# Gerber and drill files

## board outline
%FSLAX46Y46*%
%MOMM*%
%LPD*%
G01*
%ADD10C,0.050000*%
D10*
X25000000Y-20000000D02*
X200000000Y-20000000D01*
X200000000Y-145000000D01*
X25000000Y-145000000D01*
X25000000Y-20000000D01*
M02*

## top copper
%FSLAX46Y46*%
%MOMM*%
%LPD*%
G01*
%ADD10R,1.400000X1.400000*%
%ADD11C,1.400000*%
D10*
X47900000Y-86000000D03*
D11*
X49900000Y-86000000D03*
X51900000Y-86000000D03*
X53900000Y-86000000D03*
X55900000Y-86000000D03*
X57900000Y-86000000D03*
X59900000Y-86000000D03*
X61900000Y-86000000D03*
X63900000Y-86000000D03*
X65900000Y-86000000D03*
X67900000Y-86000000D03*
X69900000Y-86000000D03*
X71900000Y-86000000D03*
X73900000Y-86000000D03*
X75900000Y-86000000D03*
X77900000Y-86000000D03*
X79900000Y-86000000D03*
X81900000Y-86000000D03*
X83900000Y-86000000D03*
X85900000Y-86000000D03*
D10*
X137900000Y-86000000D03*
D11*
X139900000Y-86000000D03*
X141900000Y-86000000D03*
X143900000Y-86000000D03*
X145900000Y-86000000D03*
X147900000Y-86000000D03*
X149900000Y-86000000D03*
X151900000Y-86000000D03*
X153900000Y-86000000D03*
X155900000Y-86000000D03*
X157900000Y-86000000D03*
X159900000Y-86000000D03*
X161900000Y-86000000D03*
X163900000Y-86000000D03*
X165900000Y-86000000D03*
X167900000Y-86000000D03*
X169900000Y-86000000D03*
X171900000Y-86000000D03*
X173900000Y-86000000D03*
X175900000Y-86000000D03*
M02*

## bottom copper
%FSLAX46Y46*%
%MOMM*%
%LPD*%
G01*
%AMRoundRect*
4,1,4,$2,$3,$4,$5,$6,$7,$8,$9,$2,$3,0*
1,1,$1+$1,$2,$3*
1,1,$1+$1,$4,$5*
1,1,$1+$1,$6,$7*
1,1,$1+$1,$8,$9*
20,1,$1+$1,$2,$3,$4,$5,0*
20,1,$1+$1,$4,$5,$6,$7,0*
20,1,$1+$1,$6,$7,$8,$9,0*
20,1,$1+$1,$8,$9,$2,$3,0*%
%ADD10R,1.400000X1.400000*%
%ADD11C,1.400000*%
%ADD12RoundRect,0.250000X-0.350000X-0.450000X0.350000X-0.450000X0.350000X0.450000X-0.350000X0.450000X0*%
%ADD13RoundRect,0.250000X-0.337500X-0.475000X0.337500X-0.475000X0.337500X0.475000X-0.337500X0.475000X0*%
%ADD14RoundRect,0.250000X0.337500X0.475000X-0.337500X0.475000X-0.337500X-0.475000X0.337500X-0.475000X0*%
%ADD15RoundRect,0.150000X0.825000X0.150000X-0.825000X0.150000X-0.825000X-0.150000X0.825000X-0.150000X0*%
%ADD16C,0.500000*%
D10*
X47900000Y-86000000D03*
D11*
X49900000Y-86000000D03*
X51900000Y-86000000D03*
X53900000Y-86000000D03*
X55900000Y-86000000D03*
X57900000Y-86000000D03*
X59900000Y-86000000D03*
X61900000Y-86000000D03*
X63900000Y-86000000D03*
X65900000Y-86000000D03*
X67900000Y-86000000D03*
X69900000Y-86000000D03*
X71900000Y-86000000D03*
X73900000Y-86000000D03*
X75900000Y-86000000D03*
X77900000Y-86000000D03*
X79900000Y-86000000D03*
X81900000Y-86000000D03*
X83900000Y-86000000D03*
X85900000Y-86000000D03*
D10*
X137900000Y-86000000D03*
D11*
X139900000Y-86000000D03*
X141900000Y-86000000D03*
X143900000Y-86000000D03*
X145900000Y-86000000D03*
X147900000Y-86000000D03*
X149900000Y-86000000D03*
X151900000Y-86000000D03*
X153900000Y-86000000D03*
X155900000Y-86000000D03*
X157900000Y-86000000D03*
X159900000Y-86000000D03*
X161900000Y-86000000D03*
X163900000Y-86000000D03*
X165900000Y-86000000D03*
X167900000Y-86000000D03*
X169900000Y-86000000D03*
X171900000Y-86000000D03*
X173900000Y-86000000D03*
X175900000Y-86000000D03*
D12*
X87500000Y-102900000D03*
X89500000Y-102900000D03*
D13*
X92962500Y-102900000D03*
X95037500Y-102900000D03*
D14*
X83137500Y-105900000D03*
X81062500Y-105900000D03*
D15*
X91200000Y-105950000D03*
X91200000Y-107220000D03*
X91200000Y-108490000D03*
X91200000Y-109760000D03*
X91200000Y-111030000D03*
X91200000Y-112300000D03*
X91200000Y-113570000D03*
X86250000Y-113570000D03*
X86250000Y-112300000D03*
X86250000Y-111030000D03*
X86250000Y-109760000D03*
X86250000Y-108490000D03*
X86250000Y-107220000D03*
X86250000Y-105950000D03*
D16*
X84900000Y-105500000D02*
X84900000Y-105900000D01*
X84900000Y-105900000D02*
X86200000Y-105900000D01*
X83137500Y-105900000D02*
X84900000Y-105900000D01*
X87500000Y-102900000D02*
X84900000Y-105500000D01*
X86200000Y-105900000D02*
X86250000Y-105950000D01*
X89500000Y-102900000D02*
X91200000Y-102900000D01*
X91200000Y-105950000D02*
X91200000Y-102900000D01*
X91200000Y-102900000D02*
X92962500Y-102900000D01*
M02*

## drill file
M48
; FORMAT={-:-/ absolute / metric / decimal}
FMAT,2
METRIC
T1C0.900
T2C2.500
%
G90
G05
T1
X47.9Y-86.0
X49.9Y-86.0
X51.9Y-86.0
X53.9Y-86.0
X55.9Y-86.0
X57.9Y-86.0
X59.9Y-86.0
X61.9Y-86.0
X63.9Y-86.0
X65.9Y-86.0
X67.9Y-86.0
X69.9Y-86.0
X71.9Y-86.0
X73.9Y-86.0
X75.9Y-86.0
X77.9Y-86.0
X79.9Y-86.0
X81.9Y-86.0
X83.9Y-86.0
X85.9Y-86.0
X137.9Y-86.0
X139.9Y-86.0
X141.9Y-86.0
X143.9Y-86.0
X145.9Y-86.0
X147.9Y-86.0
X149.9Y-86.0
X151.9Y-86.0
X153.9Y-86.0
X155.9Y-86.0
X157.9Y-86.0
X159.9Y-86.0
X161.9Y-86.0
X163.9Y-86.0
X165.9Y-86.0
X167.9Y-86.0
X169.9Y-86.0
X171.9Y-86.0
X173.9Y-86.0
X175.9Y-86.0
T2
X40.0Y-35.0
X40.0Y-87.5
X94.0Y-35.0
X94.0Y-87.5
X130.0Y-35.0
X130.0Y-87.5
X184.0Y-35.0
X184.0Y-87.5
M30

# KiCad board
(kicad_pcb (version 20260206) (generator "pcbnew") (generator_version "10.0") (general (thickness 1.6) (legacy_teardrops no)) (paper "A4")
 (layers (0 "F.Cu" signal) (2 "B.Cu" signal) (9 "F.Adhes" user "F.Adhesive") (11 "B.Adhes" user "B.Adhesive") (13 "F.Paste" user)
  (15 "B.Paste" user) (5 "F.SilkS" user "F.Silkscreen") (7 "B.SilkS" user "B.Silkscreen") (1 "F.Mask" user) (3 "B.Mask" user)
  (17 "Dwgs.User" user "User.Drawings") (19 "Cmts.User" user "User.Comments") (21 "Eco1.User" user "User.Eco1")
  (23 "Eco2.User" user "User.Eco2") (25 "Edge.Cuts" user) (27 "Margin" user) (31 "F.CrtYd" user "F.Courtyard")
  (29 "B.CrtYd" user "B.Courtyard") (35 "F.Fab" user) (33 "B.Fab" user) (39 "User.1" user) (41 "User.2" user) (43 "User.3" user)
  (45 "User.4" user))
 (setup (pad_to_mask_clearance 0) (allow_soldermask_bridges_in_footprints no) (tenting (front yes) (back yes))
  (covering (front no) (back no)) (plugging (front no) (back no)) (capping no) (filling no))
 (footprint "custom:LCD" (layer "F.Cu") (at 66.9 86)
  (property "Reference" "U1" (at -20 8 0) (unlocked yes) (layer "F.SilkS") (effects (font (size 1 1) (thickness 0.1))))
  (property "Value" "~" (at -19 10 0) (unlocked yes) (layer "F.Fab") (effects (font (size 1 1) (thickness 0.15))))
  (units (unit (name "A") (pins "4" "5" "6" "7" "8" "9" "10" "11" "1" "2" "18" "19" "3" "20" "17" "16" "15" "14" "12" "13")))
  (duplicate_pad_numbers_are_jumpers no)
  (pad "" np_thru_hole circle (at -26.9 -51) (size 2.5 2.5) (drill 2.5) (layers "*.Cu" "*.Mask") (thermal_bridge_angle 90))
  (pad "" np_thru_hole circle (at -26.9 1.5) (size 2.5 2.5) (drill 2.5) (layers "*.Cu" "*.Mask") (thermal_bridge_angle 90))
  (pad "" np_thru_hole circle (at 27.1 -51) (size 2.5 2.5) (drill 2.5) (layers "*.Cu" "*.Mask") (thermal_bridge_angle 90))
  (pad "" np_thru_hole circle (at 27.1 1.5) (size 2.5 2.5) (drill 2.5) (layers "*.Cu" "*.Mask") (thermal_bridge_angle 90))
  (pad "1" thru_hole rect (at -19 0) (size 1.4 1.4) (drill 0.9) (layers "*.Cu" "*.Mask") (remove_unused_layers no)
   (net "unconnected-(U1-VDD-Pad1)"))
  (pad "2" thru_hole circle (at -17 0) (size 1.4 1.4) (drill 0.9) (layers "*.Cu" "*.Mask") (remove_unused_layers no)
   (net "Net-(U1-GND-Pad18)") (thermal_bridge_angle 90))
  (pad "3" thru_hole circle (at -15 0) (size 1.4 1.4) (drill 0.9) (layers "*.Cu" "*.Mask") (remove_unused_layers no)
   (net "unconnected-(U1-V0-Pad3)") (thermal_bridge_angle 90))
  (pad "4" thru_hole circle (at -13 0) (size 1.4 1.4) (drill 0.9) (layers "*.Cu" "*.Mask") (remove_unused_layers no)
   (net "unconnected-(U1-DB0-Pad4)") (thermal_bridge_angle 90))
  (pad "5" thru_hole circle (at -11 0) (size 1.4 1.4) (drill 0.9) (layers "*.Cu" "*.Mask") (remove_unused_layers no)
   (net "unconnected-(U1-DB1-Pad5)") (thermal_bridge_angle 90))
  (pad "6" thru_hole circle (at -9 0) (size 1.4 1.4) (drill 0.9) (layers "*.Cu" "*.Mask") (remove_unused_layers no)
   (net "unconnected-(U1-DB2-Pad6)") (thermal_bridge_angle 90))
  (pad "7" thru_hole circle (at -7 0) (size 1.4 1.4) (drill 0.9) (layers "*.Cu" "*.Mask") (remove_unused_layers no)
   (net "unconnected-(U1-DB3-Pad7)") (thermal_bridge_angle 90))
  (pad "8" thru_hole circle (at -5 0) (size 1.4 1.4) (drill 0.9) (layers "*.Cu" "*.Mask") (remove_unused_layers no)
   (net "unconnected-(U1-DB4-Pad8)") (thermal_bridge_angle 90))
  (pad "9" thru_hole circle (at -3 0) (size 1.4 1.4) (drill 0.9) (layers "*.Cu" "*.Mask") (remove_unused_layers no)
   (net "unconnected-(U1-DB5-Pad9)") (thermal_bridge_angle 90))
  (pad "10" thru_hole circle (at -1 0) (size 1.4 1.4) (drill 0.9) (layers "*.Cu" "*.Mask") (remove_unused_layers no)
   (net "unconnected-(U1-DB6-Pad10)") (thermal_bridge_angle 90))
  (pad "11" thru_hole circle (at 1 0) (size 1.4 1.4) (drill 0.9) (layers "*.Cu" "*.Mask") (remove_unused_layers no)
   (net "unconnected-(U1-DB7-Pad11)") (thermal_bridge_angle 90))
  (pad "12" thru_hole circle (at 3 0) (size 1.4 1.4) (drill 0.9) (layers "*.Cu" "*.Mask") (remove_unused_layers no)
   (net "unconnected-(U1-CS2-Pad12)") (thermal_bridge_angle 90))
  (pad "13" thru_hole circle (at 5 0) (size 1.4 1.4) (drill 0.9) (layers "*.Cu" "*.Mask") (remove_unused_layers no)
   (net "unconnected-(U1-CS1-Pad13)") (thermal_bridge_angle 90))
  (pad "14" thru_hole circle (at 7 0) (size 1.4 1.4) (drill 0.9) (layers "*.Cu" "*.Mask") (remove_unused_layers no)
   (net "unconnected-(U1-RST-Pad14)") (thermal_bridge_angle 90))
  (pad "15" thru_hole circle (at 9 0) (size 1.4 1.4) (drill 0.9) (layers "*.Cu" "*.Mask") (remove_unused_layers no)
   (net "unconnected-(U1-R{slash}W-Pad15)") (thermal_bridge_angle 90))
  (pad "16" thru_hole circle (at 11 0) (size 1.4 1.4) (drill 0.9) (layers "*.Cu" "*.Mask") (remove_unused_layers no)
   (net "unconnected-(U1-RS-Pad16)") (thermal_bridge_angle 90))
  (pad "17" thru_hole circle (at 13 0) (size 1.4 1.4) (drill 0.9) (layers "*.Cu" "*.Mask") (remove_unused_layers no)
   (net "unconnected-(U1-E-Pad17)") (thermal_bridge_angle 90))
  (pad "18" thru_hole circle (at 15 0) (size 1.4 1.4) (drill 0.9) (layers "*.Cu" "*.Mask") (remove_unused_layers no)
   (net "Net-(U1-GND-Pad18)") (thermal_bridge_angle 90))
  (pad "19" thru_hole circle (at 17 0) (size 1.4 1.4) (drill 0.9) (layers "*.Cu" "*.Mask") (remove_unused_layers no)
   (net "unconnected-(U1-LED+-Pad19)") (thermal_bridge_angle 90))
  (pad "20" thru_hole circle (at 19 0) (size 1.4 1.4) (drill 0.9) (layers "*.Cu" "*.Mask") (remove_unused_layers no)
   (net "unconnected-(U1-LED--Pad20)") (thermal_bridge_angle 90)))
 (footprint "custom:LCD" (layer "F.Cu") (at 156.9 86)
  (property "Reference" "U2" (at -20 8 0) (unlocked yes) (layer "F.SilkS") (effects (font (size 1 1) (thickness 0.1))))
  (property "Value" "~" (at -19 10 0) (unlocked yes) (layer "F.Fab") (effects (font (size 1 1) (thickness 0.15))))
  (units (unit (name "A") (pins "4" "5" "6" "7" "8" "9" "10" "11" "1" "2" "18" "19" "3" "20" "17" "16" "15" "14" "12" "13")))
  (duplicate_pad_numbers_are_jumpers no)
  (pad "" np_thru_hole circle (at -26.9 -51) (size 2.5 2.5) (drill 2.5) (layers "*.Cu" "*.Mask") (thermal_bridge_angle 90))
  (pad "" np_thru_hole circle (at -26.9 1.5) (size 2.5 2.5) (drill 2.5) (layers "*.Cu" "*.Mask") (thermal_bridge_angle 90))
  (pad "" np_thru_hole circle (at 27.1 -51) (size 2.5 2.5) (drill 2.5) (layers "*.Cu" "*.Mask") (thermal_bridge_angle 90))
  (pad "" np_thru_hole circle (at 27.1 1.5) (size 2.5 2.5) (drill 2.5) (layers "*.Cu" "*.Mask") (thermal_bridge_angle 90))
  (pad "1" thru_hole rect (at -19 0) (size 1.4 1.4) (drill 0.9) (layers "*.Cu" "*.Mask") (remove_unused_layers no)
   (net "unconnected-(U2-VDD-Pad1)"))
  (pad "2" thru_hole circle (at -17 0) (size 1.4 1.4) (drill 0.9) (layers "*.Cu" "*.Mask") (remove_unused_layers no)
   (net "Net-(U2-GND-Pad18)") (thermal_bridge_angle 90))
  (pad "3" thru_hole circle (at -15 0) (size 1.4 1.4) (drill 0.9) (layers "*.Cu" "*.Mask") (remove_unused_layers no)
   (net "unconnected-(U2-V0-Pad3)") (thermal_bridge_angle 90))
  (pad "4" thru_hole circle (at -13 0) (size 1.4 1.4) (drill 0.9) (layers "*.Cu" "*.Mask") (remove_unused_layers no)
   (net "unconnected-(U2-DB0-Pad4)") (thermal_bridge_angle 90))
  (pad "5" thru_hole circle (at -11 0) (size 1.4 1.4) (drill 0.9) (layers "*.Cu" "*.Mask") (remove_unused_layers no)
   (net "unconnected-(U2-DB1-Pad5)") (thermal_bridge_angle 90))
  (pad "6" thru_hole circle (at -9 0) (size 1.4 1.4) (drill 0.9) (layers "*.Cu" "*.Mask") (remove_unused_layers no)
   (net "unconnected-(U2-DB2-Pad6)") (thermal_bridge_angle 90))
  (pad "7" thru_hole circle (at -7 0) (size 1.4 1.4) (drill 0.9) (layers "*.Cu" "*.Mask") (remove_unused_layers no)
   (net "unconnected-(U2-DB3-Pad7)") (thermal_bridge_angle 90))
  (pad "8" thru_hole circle (at -5 0) (size 1.4 1.4) (drill 0.9) (layers "*.Cu" "*.Mask") (remove_unused_layers no)
   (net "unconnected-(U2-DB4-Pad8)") (thermal_bridge_angle 90))
  (pad "9" thru_hole circle (at -3 0) (size 1.4 1.4) (drill 0.9) (layers "*.Cu" "*.Mask") (remove_unused_layers no)
   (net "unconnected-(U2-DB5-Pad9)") (thermal_bridge_angle 90))
  (pad "10" thru_hole circle (at -1 0) (size 1.4 1.4) (drill 0.9) (layers "*.Cu" "*.Mask") (remove_unused_layers no)
   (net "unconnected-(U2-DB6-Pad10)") (thermal_bridge_angle 90))
  (pad "11" thru_hole circle (at 1 0) (size 1.4 1.4) (drill 0.9) (layers "*.Cu" "*.Mask") (remove_unused_layers no)
   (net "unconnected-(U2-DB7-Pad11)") (thermal_bridge_angle 90))
  (pad "12" thru_hole circle (at 3 0) (size 1.4 1.4) (drill 0.9) (layers "*.Cu" "*.Mask") (remove_unused_layers no)
   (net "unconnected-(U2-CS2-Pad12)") (thermal_bridge_angle 90))
  (pad "13" thru_hole circle (at 5 0) (size 1.4 1.4) (drill 0.9) (layers "*.Cu" "*.Mask") (remove_unused_layers no)
   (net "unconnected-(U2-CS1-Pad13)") (thermal_bridge_angle 90))
  (pad "14" thru_hole circle (at 7 0) (size 1.4 1.4) (drill 0.9) (layers "*.Cu" "*.Mask") (remove_unused_layers no)
   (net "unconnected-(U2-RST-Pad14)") (thermal_bridge_angle 90))
  (pad "15" thru_hole circle (at 9 0) (size 1.4 1.4) (drill 0.9) (layers "*.Cu" "*.Mask") (remove_unused_layers no)
   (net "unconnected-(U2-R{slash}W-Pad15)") (thermal_bridge_angle 90))
  (pad "16" thru_hole circle (at 11 0) (size 1.4 1.4) (drill 0.9) (layers "*.Cu" "*.Mask") (remove_unused_layers no)
   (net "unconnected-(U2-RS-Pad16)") (thermal_bridge_angle 90))
  (pad "17" thru_hole circle (at 13 0) (size 1.4 1.4) (drill 0.9) (layers "*.Cu" "*.Mask") (remove_unused_layers no)
   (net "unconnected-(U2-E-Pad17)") (thermal_bridge_angle 90))
  (pad "18" thru_hole circle (at 15 0) (size 1.4 1.4) (drill 0.9) (layers "*.Cu" "*.Mask") (remove_unused_layers no)
   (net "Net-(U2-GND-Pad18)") (thermal_bridge_angle 90))
  (pad "19" thru_hole circle (at 17 0) (size 1.4 1.4) (drill 0.9) (layers "*.Cu" "*.Mask") (remove_unused_layers no)
   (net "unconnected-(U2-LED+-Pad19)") (thermal_bridge_angle 90))
  (pad "20" thru_hole circle (at 19 0) (size 1.4 1.4) (drill 0.9) (layers "*.Cu" "*.Mask") (remove_unused_layers no)
   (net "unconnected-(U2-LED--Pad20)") (thermal_bridge_angle 90)))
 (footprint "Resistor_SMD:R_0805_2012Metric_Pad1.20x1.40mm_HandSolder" (layer "B.Cu") (at 88.5 102.9)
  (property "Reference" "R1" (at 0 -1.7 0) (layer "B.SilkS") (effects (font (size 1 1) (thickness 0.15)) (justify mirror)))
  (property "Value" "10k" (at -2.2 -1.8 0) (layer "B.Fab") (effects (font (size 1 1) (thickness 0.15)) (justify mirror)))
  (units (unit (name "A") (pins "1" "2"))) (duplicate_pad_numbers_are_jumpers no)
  (pad "1" smd roundrect (at -1 0) (size 1.2 1.4) (layers "B.Cu" "B.Mask" "B.Paste") (roundrect_rratio 0.208333) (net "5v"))
  (pad "2" smd roundrect (at 1 0) (size 1.2 1.4) (layers "B.Cu" "B.Mask" "B.Paste") (roundrect_rratio 0.208333) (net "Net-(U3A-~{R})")))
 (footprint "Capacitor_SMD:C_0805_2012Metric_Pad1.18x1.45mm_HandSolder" (layer "B.Cu") (at 94 102.9)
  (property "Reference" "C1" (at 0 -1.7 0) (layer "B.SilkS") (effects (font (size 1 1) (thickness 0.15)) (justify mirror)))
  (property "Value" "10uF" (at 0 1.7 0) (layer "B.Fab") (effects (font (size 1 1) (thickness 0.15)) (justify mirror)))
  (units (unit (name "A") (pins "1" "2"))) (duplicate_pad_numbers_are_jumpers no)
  (pad "1" smd roundrect (at -1.0375 0) (size 1.175 1.45) (layers "B.Cu" "B.Mask" "B.Paste") (roundrect_rratio 0.212766)
   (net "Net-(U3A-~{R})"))
  (pad "2" smd roundrect (at 1.0375 0) (size 1.175 1.45) (layers "B.Cu" "B.Mask" "B.Paste") (roundrect_rratio 0.212766) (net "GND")))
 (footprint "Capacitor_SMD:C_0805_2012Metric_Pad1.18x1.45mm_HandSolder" (layer "B.Cu") (at 82.1 105.9 180)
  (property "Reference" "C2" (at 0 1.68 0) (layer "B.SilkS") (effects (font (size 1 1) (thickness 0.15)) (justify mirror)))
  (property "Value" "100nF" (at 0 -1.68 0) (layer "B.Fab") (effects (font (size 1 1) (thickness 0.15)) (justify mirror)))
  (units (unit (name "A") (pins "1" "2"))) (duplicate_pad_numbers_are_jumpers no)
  (pad "1" smd roundrect (at -1.0375 0 180) (size 1.175 1.45) (layers "B.Cu" "B.Mask" "B.Paste") (roundrect_rratio 0.212766) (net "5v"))
  (pad "2" smd roundrect (at 1.0375 0 180) (size 1.175 1.45) (layers "B.Cu" "B.Mask" "B.Paste") (roundrect_rratio 0.212766) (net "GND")))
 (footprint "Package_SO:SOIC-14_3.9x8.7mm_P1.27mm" (layer "B.Cu") (at 88.725 109.76 180)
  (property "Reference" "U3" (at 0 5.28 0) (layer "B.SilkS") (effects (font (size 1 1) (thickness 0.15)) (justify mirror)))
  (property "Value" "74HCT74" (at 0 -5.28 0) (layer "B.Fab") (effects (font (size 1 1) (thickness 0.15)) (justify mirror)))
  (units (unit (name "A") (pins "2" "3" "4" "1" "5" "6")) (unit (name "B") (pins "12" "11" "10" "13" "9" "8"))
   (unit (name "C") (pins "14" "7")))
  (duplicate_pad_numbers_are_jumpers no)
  (pad "1" smd roundrect (at -2.475 3.81 180) (size 1.95 0.6) (layers "B.Cu" "B.Mask" "B.Paste") (roundrect_rratio 0.25)
   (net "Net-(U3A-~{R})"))
  (pad "2" smd roundrect (at -2.475 2.54 180) (size 1.95 0.6) (layers "B.Cu" "B.Mask" "B.Paste") (roundrect_rratio 0.25) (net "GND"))
  (pad "3" smd roundrect (at -2.475 1.27 180) (size 1.95 0.6) (layers "B.Cu" "B.Mask" "B.Paste") (roundrect_rratio 0.25) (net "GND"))
  (pad "4" smd roundrect (at -2.475 0 180) (size 1.95 0.6) (layers "B.Cu" "B.Mask" "B.Paste") (roundrect_rratio 0.25)
   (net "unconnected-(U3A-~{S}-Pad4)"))
  (pad "5" smd roundrect (at -2.475 -1.27 180) (size 1.95 0.6) (layers "B.Cu" "B.Mask" "B.Paste") (roundrect_rratio 0.25)
   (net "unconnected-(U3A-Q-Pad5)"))
  (pad "6" smd roundrect (at -2.475 -2.54 180) (size 1.95 0.6) (layers "B.Cu" "B.Mask" "B.Paste") (roundrect_rratio 0.25) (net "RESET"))
  (pad "7" smd roundrect (at -2.475 -3.81 180) (size 1.95 0.6) (layers "B.Cu" "B.Mask" "B.Paste") (roundrect_rratio 0.25) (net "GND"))
  (pad "8" smd roundrect (at 2.475 -3.81 180) (size 1.95 0.6) (layers "B.Cu" "B.Mask" "B.Paste") (roundrect_rratio 0.25)
   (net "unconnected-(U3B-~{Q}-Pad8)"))
  (pad "9" smd roundrect (at 2.475 -2.54 180) (size 1.95 0.6) (layers "B.Cu" "B.Mask" "B.Paste") (roundrect_rratio 0.25)
   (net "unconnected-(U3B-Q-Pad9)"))
  (pad "10" smd roundrect (at 2.475 -1.27 180) (size 1.95 0.6) (layers "B.Cu" "B.Mask" "B.Paste") (roundrect_rratio 0.25)
   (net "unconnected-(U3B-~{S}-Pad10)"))
  (pad "11" smd roundrect (at 2.475 0 180) (size 1.95 0.6) (layers "B.Cu" "B.Mask" "B.Paste") (roundrect_rratio 0.25)
   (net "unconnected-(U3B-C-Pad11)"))
  (pad "12" smd roundrect (at 2.475 1.27 180) (size 1.95 0.6) (layers "B.Cu" "B.Mask" "B.Paste") (roundrect_rratio 0.25)
   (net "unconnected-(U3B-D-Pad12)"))
  (pad "13" smd roundrect (at 2.475 2.54 180) (size 1.95 0.6) (layers "B.Cu" "B.Mask" "B.Paste") (roundrect_rratio 0.25)
   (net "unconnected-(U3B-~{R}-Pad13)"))
  (pad "14" smd roundrect (at 2.475 3.81 180) (size 1.95 0.6) (layers "B.Cu" "B.Mask" "B.Paste") (roundrect_rratio 0.25) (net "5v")))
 (gr_rect (start 25 20) (end 200 145) (stroke (width 0.05) (type default)) (fill no) (layer "Edge.Cuts"))
 (segment (start 84.9 105.5) (end 84.9 105.9) (width 0.5) (layer "B.Cu") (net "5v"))
 (segment (start 84.9 105.9) (end 86.2 105.9) (width 0.5) (layer "B.Cu") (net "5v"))
 (segment (start 83.1375 105.9) (end 84.9 105.9) (width 0.5) (layer "B.Cu") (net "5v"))
 (segment (start 87.5 102.9) (end 84.9 105.5) (width 0.5) (layer "B.Cu") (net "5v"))
 (segment (start 86.2 105.9) (end 86.25 105.95) (width 0.5) (layer "B.Cu") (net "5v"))
 (segment (start 89.5 102.9) (end 91.2 102.9) (width 0.5) (layer "B.Cu") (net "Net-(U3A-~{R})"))
 (segment (start 91.2 105.95) (end 91.2 102.9) (width 0.5) (layer "B.Cu") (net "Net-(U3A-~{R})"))
 (segment (start 91.2 102.9) (end 92.9625 102.9) (width 0.5) (layer "B.Cu") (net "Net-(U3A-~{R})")))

